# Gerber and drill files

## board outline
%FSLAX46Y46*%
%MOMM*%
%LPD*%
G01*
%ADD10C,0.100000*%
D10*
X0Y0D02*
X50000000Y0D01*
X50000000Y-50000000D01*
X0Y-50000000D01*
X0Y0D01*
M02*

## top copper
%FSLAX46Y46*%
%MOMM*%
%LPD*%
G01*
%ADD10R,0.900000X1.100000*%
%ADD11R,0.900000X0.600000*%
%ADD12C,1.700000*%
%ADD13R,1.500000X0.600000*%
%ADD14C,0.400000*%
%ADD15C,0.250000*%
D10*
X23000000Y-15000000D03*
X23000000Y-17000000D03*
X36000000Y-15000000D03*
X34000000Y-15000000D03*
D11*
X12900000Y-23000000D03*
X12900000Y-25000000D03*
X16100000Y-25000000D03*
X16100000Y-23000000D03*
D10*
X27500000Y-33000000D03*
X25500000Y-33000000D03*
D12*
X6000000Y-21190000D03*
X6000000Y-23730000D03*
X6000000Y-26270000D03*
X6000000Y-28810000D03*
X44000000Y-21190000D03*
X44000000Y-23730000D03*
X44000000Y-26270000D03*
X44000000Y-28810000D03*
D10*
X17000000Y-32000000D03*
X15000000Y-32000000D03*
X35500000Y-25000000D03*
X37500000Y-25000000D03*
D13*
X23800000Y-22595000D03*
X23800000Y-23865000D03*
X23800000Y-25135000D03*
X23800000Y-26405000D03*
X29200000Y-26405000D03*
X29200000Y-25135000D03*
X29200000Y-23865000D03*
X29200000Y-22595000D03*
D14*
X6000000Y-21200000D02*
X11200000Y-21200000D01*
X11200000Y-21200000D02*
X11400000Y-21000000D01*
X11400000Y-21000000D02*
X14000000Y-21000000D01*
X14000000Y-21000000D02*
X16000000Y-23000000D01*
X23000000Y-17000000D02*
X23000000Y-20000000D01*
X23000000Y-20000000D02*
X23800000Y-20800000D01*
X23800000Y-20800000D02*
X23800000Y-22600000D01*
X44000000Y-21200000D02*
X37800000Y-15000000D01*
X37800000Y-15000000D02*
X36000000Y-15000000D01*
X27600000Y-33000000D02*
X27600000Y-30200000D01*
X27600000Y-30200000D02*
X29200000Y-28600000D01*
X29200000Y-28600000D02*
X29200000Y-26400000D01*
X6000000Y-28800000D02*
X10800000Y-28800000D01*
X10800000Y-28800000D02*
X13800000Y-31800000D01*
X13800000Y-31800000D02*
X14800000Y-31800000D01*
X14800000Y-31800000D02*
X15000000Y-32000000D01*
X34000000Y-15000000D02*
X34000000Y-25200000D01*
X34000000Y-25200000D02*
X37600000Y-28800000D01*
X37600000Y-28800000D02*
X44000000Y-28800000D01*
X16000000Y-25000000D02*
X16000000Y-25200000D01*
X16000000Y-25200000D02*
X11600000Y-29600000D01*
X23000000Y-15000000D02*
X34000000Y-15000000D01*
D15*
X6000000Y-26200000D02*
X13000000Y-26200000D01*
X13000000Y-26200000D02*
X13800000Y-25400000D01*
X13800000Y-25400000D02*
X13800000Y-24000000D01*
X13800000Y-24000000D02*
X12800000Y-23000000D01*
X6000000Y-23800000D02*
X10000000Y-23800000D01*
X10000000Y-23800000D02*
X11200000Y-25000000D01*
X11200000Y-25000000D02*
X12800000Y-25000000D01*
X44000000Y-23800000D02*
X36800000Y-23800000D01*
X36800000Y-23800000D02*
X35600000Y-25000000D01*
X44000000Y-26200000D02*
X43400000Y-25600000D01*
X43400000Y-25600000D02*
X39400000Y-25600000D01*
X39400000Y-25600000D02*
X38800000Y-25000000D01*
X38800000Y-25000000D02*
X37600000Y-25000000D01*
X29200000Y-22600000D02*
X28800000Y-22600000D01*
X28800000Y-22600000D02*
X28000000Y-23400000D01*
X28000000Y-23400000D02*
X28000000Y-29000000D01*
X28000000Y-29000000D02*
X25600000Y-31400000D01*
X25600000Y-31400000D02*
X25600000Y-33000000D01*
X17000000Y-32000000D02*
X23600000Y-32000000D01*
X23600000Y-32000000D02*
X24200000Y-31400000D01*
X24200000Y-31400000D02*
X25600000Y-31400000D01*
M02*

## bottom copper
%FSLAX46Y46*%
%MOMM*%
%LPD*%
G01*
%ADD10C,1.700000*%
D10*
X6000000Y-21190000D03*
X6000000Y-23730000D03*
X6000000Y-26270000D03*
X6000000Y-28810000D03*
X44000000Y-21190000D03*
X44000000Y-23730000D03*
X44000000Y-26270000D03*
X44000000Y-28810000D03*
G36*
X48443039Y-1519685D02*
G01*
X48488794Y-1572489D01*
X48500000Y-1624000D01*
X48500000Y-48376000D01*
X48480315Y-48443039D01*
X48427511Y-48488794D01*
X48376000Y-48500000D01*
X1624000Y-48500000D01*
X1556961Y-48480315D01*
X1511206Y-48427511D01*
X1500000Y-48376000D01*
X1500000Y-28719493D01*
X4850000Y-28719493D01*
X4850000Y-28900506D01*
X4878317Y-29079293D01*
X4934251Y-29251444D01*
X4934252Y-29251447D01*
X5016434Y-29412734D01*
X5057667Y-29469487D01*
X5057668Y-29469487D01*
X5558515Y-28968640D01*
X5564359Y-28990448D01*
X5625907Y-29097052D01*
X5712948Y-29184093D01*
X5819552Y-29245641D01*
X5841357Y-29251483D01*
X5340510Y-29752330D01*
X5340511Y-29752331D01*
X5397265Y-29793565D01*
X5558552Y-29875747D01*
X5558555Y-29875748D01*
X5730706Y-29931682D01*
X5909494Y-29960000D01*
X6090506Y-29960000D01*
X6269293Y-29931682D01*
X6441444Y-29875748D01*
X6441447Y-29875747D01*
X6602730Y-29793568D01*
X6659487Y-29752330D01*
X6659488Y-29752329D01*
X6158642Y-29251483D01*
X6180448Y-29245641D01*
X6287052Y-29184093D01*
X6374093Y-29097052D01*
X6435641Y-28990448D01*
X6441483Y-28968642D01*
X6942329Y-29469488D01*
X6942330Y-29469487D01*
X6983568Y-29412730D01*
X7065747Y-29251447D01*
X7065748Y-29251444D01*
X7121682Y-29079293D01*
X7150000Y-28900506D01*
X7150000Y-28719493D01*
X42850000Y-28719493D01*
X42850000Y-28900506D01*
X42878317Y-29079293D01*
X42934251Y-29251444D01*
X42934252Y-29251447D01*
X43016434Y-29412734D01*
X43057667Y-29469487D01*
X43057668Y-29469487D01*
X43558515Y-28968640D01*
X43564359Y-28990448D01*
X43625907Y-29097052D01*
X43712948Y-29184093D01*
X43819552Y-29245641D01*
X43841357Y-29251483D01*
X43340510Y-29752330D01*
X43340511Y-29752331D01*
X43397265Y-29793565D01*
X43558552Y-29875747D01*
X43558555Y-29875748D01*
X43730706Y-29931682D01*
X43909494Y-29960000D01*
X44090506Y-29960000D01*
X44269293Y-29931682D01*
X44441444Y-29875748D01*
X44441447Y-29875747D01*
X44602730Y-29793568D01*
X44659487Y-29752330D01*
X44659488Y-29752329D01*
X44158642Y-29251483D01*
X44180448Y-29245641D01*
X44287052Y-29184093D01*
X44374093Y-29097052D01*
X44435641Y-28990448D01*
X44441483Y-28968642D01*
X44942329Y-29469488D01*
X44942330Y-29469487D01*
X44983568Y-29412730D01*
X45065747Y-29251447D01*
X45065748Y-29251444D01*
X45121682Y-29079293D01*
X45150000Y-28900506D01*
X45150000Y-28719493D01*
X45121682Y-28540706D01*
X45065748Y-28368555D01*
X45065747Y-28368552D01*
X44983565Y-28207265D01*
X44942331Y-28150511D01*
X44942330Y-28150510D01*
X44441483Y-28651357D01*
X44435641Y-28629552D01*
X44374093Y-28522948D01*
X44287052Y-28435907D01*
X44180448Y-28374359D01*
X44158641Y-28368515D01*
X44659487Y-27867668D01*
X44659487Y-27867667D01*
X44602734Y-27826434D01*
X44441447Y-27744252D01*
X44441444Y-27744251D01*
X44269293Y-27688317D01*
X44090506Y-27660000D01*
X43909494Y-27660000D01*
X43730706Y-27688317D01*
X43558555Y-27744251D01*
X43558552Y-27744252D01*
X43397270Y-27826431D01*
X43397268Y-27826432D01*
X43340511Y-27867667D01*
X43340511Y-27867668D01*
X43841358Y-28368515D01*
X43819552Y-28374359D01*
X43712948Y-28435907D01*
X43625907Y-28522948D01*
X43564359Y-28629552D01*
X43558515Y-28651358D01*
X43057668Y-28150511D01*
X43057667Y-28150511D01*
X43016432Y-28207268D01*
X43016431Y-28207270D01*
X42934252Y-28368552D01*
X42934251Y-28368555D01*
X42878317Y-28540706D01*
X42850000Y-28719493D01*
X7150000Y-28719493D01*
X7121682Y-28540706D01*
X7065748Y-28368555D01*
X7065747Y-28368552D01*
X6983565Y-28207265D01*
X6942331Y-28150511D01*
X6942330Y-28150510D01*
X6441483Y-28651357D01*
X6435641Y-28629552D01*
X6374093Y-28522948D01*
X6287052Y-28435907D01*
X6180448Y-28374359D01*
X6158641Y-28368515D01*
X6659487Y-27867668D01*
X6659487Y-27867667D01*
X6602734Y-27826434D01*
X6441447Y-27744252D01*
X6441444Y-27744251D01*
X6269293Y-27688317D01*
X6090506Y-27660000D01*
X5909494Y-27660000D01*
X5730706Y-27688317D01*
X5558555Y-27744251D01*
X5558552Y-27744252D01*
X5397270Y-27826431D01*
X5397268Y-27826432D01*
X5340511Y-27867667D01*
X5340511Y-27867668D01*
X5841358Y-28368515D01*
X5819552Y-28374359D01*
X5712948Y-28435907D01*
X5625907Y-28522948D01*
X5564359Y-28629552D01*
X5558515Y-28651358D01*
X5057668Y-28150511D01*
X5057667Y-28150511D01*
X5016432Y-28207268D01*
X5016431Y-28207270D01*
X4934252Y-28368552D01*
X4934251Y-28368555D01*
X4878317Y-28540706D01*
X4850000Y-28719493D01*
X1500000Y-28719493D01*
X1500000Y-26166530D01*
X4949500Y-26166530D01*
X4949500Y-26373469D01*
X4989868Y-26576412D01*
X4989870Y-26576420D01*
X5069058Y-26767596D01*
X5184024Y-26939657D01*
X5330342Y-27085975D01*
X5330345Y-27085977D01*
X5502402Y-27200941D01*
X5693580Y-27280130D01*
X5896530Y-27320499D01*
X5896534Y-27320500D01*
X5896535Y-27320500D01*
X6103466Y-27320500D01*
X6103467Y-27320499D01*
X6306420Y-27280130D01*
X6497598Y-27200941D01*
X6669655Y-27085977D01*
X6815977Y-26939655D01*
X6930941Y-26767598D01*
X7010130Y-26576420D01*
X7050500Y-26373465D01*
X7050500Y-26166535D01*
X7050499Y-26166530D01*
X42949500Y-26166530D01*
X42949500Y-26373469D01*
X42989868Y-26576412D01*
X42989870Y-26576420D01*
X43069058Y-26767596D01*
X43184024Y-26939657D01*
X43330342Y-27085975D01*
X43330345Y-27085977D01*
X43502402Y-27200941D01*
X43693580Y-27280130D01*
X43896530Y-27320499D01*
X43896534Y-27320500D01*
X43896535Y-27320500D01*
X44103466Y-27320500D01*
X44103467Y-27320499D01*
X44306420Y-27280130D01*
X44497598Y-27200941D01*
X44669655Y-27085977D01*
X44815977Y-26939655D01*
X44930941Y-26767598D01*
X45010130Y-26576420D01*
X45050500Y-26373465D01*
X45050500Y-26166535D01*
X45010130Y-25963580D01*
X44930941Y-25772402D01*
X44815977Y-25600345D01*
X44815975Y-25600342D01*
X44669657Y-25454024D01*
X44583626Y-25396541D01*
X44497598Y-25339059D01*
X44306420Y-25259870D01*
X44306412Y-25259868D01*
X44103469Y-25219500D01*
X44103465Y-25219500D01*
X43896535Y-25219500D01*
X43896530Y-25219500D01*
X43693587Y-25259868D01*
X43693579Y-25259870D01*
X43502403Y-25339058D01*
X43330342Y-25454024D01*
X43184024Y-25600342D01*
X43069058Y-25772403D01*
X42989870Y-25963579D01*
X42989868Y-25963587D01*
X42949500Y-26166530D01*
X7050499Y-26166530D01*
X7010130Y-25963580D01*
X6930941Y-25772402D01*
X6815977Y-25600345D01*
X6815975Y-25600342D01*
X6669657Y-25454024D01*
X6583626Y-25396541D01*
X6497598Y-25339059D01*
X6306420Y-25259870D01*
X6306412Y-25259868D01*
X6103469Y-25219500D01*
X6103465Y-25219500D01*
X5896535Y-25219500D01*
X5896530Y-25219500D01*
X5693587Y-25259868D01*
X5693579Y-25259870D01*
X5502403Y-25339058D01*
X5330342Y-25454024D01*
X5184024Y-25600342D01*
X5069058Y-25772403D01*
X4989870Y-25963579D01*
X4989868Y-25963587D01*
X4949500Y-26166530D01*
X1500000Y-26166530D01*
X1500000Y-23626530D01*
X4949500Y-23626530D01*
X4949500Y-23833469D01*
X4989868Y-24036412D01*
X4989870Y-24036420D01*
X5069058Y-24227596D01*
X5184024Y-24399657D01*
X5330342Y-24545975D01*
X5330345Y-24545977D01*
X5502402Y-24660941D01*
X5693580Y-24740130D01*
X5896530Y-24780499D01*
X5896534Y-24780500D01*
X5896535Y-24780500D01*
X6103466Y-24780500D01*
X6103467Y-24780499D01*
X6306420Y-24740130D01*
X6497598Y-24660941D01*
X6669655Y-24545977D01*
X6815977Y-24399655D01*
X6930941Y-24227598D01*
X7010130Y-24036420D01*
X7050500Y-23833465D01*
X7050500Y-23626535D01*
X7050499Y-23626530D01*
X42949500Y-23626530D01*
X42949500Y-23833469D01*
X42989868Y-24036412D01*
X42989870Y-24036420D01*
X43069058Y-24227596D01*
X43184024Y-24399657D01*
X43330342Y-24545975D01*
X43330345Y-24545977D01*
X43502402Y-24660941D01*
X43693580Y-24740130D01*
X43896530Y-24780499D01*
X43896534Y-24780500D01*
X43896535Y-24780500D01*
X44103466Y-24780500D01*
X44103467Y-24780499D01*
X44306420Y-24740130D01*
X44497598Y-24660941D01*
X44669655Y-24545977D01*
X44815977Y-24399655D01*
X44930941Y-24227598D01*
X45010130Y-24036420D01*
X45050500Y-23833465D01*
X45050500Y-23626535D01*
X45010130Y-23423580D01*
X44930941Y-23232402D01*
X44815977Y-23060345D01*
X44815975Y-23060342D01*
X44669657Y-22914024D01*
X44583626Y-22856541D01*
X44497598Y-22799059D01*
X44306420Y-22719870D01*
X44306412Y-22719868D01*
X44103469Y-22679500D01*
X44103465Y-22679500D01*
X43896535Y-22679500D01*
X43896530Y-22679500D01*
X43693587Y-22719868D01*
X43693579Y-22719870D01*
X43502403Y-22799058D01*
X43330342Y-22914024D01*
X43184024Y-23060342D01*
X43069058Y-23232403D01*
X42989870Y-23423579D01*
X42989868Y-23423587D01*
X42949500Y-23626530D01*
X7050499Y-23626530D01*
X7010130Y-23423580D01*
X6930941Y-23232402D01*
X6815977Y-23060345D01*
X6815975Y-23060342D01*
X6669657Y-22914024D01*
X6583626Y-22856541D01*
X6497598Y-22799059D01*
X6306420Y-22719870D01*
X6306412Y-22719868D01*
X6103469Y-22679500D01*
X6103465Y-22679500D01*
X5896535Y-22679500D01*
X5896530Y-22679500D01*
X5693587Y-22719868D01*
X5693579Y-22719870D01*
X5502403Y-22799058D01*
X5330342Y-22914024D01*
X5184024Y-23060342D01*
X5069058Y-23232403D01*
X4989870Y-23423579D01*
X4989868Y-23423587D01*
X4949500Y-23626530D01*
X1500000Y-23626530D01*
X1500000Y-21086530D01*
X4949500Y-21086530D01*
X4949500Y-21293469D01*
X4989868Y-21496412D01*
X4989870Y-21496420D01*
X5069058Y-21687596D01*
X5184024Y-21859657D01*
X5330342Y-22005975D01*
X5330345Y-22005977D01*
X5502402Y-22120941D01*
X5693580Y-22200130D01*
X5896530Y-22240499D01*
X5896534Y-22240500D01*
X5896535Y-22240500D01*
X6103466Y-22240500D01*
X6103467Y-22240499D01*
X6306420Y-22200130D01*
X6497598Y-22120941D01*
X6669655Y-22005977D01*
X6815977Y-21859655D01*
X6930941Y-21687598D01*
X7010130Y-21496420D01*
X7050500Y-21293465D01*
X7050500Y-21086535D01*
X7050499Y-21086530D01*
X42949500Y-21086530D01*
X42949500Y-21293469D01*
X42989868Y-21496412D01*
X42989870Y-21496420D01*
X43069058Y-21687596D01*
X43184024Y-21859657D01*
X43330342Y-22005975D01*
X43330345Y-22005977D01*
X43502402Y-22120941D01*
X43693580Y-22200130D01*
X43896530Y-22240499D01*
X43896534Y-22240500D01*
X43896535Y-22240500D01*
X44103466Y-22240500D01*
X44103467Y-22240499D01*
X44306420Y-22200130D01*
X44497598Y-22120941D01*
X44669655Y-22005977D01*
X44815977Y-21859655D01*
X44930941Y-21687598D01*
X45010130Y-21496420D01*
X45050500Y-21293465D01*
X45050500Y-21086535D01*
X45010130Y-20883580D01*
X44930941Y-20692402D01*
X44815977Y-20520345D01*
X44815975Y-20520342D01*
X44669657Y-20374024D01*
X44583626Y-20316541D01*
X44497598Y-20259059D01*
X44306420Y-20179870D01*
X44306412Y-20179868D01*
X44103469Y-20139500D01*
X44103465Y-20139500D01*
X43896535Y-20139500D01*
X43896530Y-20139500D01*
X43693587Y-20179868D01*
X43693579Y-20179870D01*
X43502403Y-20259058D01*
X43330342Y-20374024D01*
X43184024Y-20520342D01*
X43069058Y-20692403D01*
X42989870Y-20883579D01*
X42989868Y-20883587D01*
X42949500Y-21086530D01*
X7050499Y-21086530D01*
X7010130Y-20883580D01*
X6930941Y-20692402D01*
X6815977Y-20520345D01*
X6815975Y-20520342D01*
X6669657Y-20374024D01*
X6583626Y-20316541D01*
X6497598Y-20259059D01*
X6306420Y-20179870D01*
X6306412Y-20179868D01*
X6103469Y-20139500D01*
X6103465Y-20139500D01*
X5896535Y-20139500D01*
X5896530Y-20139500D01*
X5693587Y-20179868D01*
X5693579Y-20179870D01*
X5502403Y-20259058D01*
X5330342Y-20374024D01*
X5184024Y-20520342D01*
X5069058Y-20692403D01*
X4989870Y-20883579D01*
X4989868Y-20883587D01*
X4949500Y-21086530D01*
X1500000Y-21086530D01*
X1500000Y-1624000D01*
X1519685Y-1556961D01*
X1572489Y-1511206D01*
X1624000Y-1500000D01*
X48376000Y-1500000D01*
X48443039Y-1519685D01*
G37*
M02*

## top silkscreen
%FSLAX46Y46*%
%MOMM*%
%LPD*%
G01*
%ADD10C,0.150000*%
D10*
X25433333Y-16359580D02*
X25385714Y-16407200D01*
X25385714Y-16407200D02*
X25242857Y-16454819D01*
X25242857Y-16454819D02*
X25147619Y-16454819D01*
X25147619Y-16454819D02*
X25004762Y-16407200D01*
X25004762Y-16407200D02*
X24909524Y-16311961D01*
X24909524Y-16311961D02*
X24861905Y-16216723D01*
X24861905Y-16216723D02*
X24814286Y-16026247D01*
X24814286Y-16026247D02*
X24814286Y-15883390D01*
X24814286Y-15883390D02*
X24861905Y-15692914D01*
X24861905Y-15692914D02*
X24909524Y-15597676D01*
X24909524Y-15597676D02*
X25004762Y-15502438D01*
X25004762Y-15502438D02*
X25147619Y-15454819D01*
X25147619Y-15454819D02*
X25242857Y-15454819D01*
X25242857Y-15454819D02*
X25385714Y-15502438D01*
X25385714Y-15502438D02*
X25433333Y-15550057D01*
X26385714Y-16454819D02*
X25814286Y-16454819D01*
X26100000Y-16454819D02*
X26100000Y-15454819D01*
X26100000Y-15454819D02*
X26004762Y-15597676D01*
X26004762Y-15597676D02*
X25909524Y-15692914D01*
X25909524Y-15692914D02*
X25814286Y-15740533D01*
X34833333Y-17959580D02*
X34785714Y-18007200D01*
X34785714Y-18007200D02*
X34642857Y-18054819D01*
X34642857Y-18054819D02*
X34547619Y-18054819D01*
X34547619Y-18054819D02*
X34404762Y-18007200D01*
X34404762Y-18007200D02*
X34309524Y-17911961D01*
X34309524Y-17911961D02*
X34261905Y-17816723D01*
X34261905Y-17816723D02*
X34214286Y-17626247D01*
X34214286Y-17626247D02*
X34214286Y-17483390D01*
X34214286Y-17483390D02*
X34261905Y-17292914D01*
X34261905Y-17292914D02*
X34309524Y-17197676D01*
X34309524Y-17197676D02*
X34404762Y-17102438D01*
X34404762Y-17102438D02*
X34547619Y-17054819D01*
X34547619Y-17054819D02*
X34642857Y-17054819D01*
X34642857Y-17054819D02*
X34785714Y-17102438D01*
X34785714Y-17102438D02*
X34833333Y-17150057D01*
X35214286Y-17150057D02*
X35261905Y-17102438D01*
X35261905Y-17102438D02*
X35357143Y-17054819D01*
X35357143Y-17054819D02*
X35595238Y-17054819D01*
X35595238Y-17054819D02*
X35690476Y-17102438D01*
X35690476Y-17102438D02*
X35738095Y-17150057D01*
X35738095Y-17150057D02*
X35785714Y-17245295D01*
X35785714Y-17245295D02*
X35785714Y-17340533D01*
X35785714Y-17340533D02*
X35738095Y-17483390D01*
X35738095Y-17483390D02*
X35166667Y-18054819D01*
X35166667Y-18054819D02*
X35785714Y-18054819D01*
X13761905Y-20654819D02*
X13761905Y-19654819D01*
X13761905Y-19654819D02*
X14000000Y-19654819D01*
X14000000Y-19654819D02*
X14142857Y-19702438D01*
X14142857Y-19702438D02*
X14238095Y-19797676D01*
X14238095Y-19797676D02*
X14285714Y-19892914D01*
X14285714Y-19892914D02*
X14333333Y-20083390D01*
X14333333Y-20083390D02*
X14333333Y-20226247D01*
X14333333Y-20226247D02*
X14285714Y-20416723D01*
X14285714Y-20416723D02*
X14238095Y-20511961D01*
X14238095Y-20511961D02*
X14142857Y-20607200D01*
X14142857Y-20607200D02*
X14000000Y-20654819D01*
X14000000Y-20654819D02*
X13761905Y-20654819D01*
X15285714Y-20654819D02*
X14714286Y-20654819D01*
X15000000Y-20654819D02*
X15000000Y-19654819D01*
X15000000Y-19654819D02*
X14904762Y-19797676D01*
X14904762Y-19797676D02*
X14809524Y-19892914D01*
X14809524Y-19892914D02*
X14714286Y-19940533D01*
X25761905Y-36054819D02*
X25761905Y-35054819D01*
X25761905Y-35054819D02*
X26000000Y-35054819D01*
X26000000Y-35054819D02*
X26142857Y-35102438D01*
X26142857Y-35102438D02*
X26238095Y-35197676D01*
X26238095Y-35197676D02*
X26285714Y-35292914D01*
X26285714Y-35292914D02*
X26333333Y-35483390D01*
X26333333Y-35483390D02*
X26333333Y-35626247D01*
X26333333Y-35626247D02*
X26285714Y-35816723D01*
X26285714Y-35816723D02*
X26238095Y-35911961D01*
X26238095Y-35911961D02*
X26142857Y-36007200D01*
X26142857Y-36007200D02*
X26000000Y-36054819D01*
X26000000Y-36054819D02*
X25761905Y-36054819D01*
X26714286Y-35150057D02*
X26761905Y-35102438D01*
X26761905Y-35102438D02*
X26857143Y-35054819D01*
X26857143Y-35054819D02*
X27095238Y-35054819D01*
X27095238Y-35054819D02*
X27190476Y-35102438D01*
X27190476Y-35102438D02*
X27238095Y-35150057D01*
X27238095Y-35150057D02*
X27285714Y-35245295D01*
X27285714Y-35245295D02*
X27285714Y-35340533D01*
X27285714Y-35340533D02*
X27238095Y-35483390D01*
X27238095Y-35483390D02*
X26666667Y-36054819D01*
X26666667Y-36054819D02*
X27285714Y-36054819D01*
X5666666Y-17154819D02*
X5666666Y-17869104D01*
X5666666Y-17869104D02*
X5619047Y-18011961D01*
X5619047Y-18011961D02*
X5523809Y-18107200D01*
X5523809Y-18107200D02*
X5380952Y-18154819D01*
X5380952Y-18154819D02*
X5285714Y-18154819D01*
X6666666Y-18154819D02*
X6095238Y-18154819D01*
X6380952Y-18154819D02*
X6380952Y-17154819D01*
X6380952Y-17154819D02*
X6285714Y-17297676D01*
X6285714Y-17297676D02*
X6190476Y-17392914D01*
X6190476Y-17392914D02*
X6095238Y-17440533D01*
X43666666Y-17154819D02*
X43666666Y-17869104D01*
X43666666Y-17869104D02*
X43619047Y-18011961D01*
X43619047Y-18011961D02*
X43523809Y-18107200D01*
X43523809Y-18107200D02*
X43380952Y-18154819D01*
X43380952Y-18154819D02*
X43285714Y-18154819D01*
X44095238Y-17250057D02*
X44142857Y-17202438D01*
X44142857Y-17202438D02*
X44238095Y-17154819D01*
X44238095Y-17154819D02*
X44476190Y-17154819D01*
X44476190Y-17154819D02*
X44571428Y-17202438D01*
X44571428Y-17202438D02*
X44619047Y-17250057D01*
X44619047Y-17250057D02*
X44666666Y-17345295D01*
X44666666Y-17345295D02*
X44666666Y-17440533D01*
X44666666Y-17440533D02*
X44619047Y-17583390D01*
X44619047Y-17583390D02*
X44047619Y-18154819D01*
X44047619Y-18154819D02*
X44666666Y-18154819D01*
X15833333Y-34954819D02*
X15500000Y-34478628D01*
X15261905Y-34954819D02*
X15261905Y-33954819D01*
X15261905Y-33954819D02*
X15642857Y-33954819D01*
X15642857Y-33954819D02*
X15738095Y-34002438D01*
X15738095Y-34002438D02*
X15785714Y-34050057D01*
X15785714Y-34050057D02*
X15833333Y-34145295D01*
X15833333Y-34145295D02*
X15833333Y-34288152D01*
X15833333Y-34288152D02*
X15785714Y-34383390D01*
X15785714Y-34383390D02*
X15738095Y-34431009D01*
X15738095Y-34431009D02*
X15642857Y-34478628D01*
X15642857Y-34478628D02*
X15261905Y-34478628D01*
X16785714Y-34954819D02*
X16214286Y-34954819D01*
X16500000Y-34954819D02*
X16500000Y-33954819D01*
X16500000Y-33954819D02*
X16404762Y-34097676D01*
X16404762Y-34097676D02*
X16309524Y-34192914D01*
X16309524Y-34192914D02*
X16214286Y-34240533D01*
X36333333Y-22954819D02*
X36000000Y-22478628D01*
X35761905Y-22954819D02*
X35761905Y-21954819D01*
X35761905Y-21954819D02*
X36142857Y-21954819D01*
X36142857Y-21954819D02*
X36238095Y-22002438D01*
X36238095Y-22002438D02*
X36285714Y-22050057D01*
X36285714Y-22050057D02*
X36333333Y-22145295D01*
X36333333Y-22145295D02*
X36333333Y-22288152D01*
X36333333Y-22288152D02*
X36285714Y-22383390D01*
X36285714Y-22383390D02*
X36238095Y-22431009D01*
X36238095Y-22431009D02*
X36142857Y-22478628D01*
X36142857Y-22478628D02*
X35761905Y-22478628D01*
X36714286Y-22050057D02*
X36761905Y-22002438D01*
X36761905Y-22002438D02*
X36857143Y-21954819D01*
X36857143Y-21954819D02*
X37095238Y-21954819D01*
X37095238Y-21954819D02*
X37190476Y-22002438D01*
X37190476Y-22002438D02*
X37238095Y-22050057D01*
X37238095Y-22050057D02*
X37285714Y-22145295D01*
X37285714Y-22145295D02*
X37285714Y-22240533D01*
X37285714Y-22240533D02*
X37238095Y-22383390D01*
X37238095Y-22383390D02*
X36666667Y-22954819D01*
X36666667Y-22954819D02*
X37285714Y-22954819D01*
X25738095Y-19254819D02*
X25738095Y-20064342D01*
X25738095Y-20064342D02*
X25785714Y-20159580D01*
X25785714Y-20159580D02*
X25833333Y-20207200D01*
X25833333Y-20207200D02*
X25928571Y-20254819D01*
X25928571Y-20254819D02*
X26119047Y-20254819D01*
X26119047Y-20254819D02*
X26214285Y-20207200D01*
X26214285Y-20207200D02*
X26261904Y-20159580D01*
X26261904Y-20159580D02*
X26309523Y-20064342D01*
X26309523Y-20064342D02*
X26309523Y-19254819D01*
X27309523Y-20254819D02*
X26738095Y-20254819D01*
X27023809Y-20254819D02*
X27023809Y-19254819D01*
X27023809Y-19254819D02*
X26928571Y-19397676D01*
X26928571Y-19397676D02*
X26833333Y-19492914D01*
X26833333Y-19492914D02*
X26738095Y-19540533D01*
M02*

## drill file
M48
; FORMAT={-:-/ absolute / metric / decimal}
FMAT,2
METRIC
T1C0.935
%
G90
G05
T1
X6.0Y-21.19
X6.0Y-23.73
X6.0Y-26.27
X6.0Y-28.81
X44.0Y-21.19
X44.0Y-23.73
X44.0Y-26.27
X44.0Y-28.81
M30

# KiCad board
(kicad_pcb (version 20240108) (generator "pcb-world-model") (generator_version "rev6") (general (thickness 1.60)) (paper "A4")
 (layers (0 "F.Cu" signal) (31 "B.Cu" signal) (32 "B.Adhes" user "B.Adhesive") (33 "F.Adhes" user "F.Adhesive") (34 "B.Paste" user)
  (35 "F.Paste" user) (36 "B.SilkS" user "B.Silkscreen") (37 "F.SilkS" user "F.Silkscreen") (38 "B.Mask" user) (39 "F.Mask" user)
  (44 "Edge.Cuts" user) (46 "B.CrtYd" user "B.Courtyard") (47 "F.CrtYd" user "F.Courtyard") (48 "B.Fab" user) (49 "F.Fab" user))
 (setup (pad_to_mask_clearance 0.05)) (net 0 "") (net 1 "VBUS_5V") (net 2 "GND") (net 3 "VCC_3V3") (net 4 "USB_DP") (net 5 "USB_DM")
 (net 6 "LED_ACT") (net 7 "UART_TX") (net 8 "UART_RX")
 (gr_rect (start 0.0 0.0) (end 50.0000 50.0000) (stroke (width 0.1) (type default)) (fill none) (layer "Edge.Cuts"))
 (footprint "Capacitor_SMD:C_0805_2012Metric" (layer "F.Cu") (at 23.0000 16.0000 270)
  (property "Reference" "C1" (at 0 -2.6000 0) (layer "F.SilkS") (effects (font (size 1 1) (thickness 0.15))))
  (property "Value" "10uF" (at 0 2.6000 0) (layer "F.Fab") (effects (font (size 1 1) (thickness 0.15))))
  (pad "1" smd rect (at -1.0000 0.0000) (size 0.9000 1.1000) (layers "F.Cu" "F.Paste" "F.Mask") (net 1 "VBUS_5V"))
  (pad "2" smd rect (at 1.0000 0.0000) (size 0.9000 1.1000) (layers "F.Cu" "F.Paste" "F.Mask") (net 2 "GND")))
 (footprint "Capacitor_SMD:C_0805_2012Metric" (layer "F.Cu") (at 35.0000 15.0000 180)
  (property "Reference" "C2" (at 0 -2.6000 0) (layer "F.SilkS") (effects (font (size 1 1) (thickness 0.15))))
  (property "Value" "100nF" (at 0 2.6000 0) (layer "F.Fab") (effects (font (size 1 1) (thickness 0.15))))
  (pad "1" smd rect (at -1.0000 0.0000) (size 0.9000 1.1000) (layers "F.Cu" "F.Paste" "F.Mask") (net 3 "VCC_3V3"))
  (pad "2" smd rect (at 1.0000 0.0000) (size 0.9000 1.1000) (layers "F.Cu" "F.Paste" "F.Mask") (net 2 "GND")))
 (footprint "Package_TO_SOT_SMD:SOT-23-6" (layer "F.Cu") (at 14.5000 24.0000 0)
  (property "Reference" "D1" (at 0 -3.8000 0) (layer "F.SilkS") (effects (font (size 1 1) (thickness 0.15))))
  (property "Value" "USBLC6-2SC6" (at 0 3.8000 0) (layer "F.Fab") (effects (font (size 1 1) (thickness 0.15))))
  (pad "1" smd rect (at -1.6000 -1.0000) (size 0.9000 0.6000) (layers "F.Cu" "F.Paste" "F.Mask") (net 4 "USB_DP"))
  (pad "2" smd rect (at -1.6000 1.0000) (size 0.9000 0.6000) (layers "F.Cu" "F.Paste" "F.Mask") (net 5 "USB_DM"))
  (pad "3" smd rect (at 1.6000 1.0000) (size 0.9000 0.6000) (layers "F.Cu" "F.Paste" "F.Mask") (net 2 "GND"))
  (pad "4" smd rect (at 1.6000 -1.0000) (size 0.9000 0.6000) (layers "F.Cu" "F.Paste" "F.Mask") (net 1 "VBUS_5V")))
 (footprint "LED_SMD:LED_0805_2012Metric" (layer "F.Cu") (at 26.5000 33.0000 180)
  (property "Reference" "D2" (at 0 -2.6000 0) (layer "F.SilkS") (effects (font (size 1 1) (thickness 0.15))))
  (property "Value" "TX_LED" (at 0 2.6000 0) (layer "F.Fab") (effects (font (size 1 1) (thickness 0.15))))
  (pad "1" smd rect (at -1.0000 0.0000) (size 0.9000 1.1000) (layers "F.Cu" "F.Paste" "F.Mask") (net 3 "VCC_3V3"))
  (pad "2" smd rect (at 1.0000 0.0000) (size 0.9000 1.1000) (layers "F.Cu" "F.Paste" "F.Mask") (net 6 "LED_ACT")))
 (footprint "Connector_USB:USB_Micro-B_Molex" (layer "F.Cu") (at 6.0000 25.0000 0) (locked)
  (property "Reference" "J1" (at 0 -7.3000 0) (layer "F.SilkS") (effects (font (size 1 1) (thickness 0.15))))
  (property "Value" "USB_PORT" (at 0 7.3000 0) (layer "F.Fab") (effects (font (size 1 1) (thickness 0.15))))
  (pad "1" thru_hole circle (at 0.0000 -3.8100) (size 1.7000 1.7000) (drill 0.9350) (layers "*.Cu" "*.Mask") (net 1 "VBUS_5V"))
  (pad "2" thru_hole circle (at 0.0000 -1.2700) (size 1.7000 1.7000) (drill 0.9350) (layers "*.Cu" "*.Mask") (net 5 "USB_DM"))
  (pad "3" thru_hole circle (at 0.0000 1.2700) (size 1.7000 1.7000) (drill 0.9350) (layers "*.Cu" "*.Mask") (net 4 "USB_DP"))
  (pad "4" thru_hole circle (at 0.0000 3.8100) (size 1.7000 1.7000) (drill 0.9350) (layers "*.Cu" "*.Mask") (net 2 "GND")))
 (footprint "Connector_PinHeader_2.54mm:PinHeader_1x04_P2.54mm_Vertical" (layer "F.Cu") (at 44.0000 25.0000 0) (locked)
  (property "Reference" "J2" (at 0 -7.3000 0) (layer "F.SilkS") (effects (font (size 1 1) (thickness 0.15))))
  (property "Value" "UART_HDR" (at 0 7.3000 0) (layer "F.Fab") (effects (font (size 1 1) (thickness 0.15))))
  (pad "1" thru_hole circle (at 0.0000 -3.8100) (size 1.7000 1.7000) (drill 0.9350) (layers "*.Cu" "*.Mask") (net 3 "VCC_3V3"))
  (pad "2" thru_hole circle (at 0.0000 -1.2700) (size 1.7000 1.7000) (drill 0.9350) (layers "*.Cu" "*.Mask") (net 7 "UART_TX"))
  (pad "3" thru_hole circle (at 0.0000 1.2700) (size 1.7000 1.7000) (drill 0.9350) (layers "*.Cu" "*.Mask") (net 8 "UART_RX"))
  (pad "4" thru_hole circle (at 0.0000 3.8100) (size 1.7000 1.7000) (drill 0.9350) (layers "*.Cu" "*.Mask") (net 2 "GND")))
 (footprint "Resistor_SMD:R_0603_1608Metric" (layer "F.Cu") (at 16.0000 32.0000 180)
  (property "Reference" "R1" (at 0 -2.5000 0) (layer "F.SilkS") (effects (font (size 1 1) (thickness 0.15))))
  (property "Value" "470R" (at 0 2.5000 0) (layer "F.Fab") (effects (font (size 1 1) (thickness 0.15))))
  (pad "1" smd rect (at -1.0000 0.0000) (size 0.9000 1.1000) (layers "F.Cu" "F.Paste" "F.Mask") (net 6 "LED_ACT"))
  (pad "2" smd rect (at 1.0000 0.0000) (size 0.9000 1.1000) (layers "F.Cu" "F.Paste" "F.Mask") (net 2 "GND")))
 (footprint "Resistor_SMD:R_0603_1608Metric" (layer "F.Cu") (at 36.5000 25.0000 0)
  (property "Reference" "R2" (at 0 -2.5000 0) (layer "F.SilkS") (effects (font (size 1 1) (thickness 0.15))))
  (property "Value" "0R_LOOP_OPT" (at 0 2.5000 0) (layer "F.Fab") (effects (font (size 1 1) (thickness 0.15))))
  (pad "1" smd rect (at -1.0000 0.0000) (size 0.9000 1.1000) (layers "F.Cu" "F.Paste" "F.Mask") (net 7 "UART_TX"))
  (pad "2" smd rect (at 1.0000 0.0000) (size 0.9000 1.1000) (layers "F.Cu" "F.Paste" "F.Mask") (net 8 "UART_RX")))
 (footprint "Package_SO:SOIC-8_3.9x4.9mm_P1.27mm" (layer "F.Cu") (at 26.5000 24.5000 0)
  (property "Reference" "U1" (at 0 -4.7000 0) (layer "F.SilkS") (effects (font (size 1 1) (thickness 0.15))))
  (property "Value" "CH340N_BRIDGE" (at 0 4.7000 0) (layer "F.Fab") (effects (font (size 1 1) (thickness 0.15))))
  (pad "1" smd rect (at -2.7000 -1.9050) (size 1.5000 0.6000) (layers "F.Cu" "F.Paste" "F.Mask") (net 1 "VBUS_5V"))
  (pad "2" smd rect (at -2.7000 -0.6350) (size 1.5000 0.6000) (layers "F.Cu" "F.Paste" "F.Mask") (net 4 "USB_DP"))
  (pad "3" smd rect (at -2.7000 0.6350) (size 1.5000 0.6000) (layers "F.Cu" "F.Paste" "F.Mask") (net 5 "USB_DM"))
  (pad "4" smd rect (at -2.7000 1.9050) (size 1.5000 0.6000) (layers "F.Cu" "F.Paste" "F.Mask") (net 2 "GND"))
  (pad "5" smd rect (at 2.7000 1.9050) (size 1.5000 0.6000) (layers "F.Cu" "F.Paste" "F.Mask") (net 3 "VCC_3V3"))
  (pad "6" smd rect (at 2.7000 0.6350) (size 1.5000 0.6000) (layers "F.Cu" "F.Paste" "F.Mask") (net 7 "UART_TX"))
  (pad "7" smd rect (at 2.7000 -0.6350) (size 1.5000 0.6000) (layers "F.Cu" "F.Paste" "F.Mask") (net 8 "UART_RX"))
  (pad "8" smd rect (at 2.7000 -1.9050) (size 1.5000 0.6000) (layers "F.Cu" "F.Paste" "F.Mask") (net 6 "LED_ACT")))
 (segment (start 6.0000 21.2000) (end 11.2000 21.2000) (width 0.4000) (layer "F.Cu") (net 1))
 (segment (start 11.2000 21.2000) (end 11.4000 21.0000) (width 0.4000) (layer "F.Cu") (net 1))
 (segment (start 11.4000 21.0000) (end 14.0000 21.0000) (width 0.4000) (layer "F.Cu") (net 1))
 (segment (start 14.0000 21.0000) (end 16.0000 23.0000) (width 0.4000) (layer "F.Cu") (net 1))
 (segment (start 23.0000 17.0000) (end 23.0000 20.0000) (width 0.4000) (layer "F.Cu") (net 1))
 (segment (start 23.0000 20.0000) (end 23.8000 20.8000) (width 0.4000) (layer "F.Cu") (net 1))
 (segment (start 23.8000 20.8000) (end 23.8000 22.6000) (width 0.4000) (layer "F.Cu") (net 1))
 (segment (start 44.0000 21.2000) (end 37.8000 15.0000) (width 0.4000) (layer "F.Cu") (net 3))
 (segment (start 37.8000 15.0000) (end 36.0000 15.0000) (width 0.4000) (layer "F.Cu") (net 3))
 (segment (start 27.6000 33.0000) (end 27.6000 30.2000) (width 0.4000) (layer "F.Cu") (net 3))
 (segment (start 27.6000 30.2000) (end 29.2000 28.6000) (width 0.4000) (layer "F.Cu") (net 3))
 (segment (start 29.2000 28.6000) (end 29.2000 26.4000) (width 0.4000) (layer "F.Cu") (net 3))
 (segment (start 6.0000 28.8000) (end 10.8000 28.8000) (width 0.4000) (layer "F.Cu") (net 2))
 (segment (start 10.8000 28.8000) (end 13.8000 31.8000) (width 0.4000) (layer "F.Cu") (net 2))
 (segment (start 13.8000 31.8000) (end 14.8000 31.8000) (width 0.4000) (layer "F.Cu") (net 2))
 (segment (start 14.8000 31.8000) (end 15.0000 32.0000) (width 0.4000) (layer "F.Cu") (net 2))
 (segment (start 34.0000 15.0000) (end 34.0000 25.2000) (width 0.4000) (layer "F.Cu") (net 2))
 (segment (start 34.0000 25.2000) (end 37.6000 28.8000) (width 0.4000) (layer "F.Cu") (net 2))
 (segment (start 37.6000 28.8000) (end 44.0000 28.8000) (width 0.4000) (layer "F.Cu") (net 2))
 (segment (start 16.0000 25.0000) (end 16.0000 25.2000) (width 0.4000) (layer "F.Cu") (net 2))
 (segment (start 16.0000 25.2000) (end 11.6000 29.6000) (width 0.4000) (layer "F.Cu") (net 2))
 (segment (start 23.0000 15.0000) (end 34.0000 15.0000) (width 0.4000) (layer "F.Cu") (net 2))
 (segment (start 6.0000 26.2000) (end 13.0000 26.2000) (width 0.2500) (layer "F.Cu") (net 4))
 (segment (start 13.0000 26.2000) (end 13.8000 25.4000) (width 0.2500) (layer "F.Cu") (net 4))
 (segment (start 13.8000 25.4000) (end 13.8000 24.0000) (width 0.2500) (layer "F.Cu") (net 4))
 (segment (start 13.8000 24.0000) (end 12.8000 23.0000) (width 0.2500) (layer "F.Cu") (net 4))
 (segment (start 6.0000 23.8000) (end 10.0000 23.8000) (width 0.2500) (layer "F.Cu") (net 5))
 (segment (start 10.0000 23.8000) (end 11.2000 25.0000) (width 0.2500) (layer "F.Cu") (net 5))
 (segment (start 11.2000 25.0000) (end 12.8000 25.0000) (width 0.2500) (layer "F.Cu") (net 5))
 (segment (start 44.0000 23.8000) (end 36.8000 23.8000) (width 0.2500) (layer "F.Cu") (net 7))
 (segment (start 36.8000 23.8000) (end 35.6000 25.0000) (width 0.2500) (layer "F.Cu") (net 7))
 (segment (start 44.0000 26.2000) (end 43.4000 25.6000) (width 0.2500) (layer "F.Cu") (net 8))
 (segment (start 43.4000 25.6000) (end 39.4000 25.6000) (width 0.2500) (layer "F.Cu") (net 8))
 (segment (start 39.4000 25.6000) (end 38.8000 25.0000) (width 0.2500) (layer "F.Cu") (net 8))
 (segment (start 38.8000 25.0000) (end 37.6000 25.0000) (width 0.2500) (layer "F.Cu") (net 8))
 (segment (start 29.2000 22.6000) (end 28.8000 22.6000) (width 0.2500) (layer "F.Cu") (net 6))
 (segment (start 28.8000 22.6000) (end 28.0000 23.4000) (width 0.2500) (layer "F.Cu") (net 6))
 (segment (start 28.0000 23.4000) (end 28.0000 29.0000) (width 0.2500) (layer "F.Cu") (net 6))
 (segment (start 28.0000 29.0000) (end 25.6000 31.4000) (width 0.2500) (layer "F.Cu") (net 6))
 (segment (start 25.6000 31.4000) (end 25.6000 33.0000) (width 0.2500) (layer "F.Cu") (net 6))
 (segment (start 17.0000 32.0000) (end 23.6000 32.0000) (width 0.2500) (layer "F.Cu") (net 6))
 (segment (start 23.6000 32.0000) (end 24.2000 31.4000) (width 0.2500) (layer "F.Cu") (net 6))
 (segment (start 24.2000 31.4000) (end 25.6000 31.4000) (width 0.2500) (layer "F.Cu") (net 6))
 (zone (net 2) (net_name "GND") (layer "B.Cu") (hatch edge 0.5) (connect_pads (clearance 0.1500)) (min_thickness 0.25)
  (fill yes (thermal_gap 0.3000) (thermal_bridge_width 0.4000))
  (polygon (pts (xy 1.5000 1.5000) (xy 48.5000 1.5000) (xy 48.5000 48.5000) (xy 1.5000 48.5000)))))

